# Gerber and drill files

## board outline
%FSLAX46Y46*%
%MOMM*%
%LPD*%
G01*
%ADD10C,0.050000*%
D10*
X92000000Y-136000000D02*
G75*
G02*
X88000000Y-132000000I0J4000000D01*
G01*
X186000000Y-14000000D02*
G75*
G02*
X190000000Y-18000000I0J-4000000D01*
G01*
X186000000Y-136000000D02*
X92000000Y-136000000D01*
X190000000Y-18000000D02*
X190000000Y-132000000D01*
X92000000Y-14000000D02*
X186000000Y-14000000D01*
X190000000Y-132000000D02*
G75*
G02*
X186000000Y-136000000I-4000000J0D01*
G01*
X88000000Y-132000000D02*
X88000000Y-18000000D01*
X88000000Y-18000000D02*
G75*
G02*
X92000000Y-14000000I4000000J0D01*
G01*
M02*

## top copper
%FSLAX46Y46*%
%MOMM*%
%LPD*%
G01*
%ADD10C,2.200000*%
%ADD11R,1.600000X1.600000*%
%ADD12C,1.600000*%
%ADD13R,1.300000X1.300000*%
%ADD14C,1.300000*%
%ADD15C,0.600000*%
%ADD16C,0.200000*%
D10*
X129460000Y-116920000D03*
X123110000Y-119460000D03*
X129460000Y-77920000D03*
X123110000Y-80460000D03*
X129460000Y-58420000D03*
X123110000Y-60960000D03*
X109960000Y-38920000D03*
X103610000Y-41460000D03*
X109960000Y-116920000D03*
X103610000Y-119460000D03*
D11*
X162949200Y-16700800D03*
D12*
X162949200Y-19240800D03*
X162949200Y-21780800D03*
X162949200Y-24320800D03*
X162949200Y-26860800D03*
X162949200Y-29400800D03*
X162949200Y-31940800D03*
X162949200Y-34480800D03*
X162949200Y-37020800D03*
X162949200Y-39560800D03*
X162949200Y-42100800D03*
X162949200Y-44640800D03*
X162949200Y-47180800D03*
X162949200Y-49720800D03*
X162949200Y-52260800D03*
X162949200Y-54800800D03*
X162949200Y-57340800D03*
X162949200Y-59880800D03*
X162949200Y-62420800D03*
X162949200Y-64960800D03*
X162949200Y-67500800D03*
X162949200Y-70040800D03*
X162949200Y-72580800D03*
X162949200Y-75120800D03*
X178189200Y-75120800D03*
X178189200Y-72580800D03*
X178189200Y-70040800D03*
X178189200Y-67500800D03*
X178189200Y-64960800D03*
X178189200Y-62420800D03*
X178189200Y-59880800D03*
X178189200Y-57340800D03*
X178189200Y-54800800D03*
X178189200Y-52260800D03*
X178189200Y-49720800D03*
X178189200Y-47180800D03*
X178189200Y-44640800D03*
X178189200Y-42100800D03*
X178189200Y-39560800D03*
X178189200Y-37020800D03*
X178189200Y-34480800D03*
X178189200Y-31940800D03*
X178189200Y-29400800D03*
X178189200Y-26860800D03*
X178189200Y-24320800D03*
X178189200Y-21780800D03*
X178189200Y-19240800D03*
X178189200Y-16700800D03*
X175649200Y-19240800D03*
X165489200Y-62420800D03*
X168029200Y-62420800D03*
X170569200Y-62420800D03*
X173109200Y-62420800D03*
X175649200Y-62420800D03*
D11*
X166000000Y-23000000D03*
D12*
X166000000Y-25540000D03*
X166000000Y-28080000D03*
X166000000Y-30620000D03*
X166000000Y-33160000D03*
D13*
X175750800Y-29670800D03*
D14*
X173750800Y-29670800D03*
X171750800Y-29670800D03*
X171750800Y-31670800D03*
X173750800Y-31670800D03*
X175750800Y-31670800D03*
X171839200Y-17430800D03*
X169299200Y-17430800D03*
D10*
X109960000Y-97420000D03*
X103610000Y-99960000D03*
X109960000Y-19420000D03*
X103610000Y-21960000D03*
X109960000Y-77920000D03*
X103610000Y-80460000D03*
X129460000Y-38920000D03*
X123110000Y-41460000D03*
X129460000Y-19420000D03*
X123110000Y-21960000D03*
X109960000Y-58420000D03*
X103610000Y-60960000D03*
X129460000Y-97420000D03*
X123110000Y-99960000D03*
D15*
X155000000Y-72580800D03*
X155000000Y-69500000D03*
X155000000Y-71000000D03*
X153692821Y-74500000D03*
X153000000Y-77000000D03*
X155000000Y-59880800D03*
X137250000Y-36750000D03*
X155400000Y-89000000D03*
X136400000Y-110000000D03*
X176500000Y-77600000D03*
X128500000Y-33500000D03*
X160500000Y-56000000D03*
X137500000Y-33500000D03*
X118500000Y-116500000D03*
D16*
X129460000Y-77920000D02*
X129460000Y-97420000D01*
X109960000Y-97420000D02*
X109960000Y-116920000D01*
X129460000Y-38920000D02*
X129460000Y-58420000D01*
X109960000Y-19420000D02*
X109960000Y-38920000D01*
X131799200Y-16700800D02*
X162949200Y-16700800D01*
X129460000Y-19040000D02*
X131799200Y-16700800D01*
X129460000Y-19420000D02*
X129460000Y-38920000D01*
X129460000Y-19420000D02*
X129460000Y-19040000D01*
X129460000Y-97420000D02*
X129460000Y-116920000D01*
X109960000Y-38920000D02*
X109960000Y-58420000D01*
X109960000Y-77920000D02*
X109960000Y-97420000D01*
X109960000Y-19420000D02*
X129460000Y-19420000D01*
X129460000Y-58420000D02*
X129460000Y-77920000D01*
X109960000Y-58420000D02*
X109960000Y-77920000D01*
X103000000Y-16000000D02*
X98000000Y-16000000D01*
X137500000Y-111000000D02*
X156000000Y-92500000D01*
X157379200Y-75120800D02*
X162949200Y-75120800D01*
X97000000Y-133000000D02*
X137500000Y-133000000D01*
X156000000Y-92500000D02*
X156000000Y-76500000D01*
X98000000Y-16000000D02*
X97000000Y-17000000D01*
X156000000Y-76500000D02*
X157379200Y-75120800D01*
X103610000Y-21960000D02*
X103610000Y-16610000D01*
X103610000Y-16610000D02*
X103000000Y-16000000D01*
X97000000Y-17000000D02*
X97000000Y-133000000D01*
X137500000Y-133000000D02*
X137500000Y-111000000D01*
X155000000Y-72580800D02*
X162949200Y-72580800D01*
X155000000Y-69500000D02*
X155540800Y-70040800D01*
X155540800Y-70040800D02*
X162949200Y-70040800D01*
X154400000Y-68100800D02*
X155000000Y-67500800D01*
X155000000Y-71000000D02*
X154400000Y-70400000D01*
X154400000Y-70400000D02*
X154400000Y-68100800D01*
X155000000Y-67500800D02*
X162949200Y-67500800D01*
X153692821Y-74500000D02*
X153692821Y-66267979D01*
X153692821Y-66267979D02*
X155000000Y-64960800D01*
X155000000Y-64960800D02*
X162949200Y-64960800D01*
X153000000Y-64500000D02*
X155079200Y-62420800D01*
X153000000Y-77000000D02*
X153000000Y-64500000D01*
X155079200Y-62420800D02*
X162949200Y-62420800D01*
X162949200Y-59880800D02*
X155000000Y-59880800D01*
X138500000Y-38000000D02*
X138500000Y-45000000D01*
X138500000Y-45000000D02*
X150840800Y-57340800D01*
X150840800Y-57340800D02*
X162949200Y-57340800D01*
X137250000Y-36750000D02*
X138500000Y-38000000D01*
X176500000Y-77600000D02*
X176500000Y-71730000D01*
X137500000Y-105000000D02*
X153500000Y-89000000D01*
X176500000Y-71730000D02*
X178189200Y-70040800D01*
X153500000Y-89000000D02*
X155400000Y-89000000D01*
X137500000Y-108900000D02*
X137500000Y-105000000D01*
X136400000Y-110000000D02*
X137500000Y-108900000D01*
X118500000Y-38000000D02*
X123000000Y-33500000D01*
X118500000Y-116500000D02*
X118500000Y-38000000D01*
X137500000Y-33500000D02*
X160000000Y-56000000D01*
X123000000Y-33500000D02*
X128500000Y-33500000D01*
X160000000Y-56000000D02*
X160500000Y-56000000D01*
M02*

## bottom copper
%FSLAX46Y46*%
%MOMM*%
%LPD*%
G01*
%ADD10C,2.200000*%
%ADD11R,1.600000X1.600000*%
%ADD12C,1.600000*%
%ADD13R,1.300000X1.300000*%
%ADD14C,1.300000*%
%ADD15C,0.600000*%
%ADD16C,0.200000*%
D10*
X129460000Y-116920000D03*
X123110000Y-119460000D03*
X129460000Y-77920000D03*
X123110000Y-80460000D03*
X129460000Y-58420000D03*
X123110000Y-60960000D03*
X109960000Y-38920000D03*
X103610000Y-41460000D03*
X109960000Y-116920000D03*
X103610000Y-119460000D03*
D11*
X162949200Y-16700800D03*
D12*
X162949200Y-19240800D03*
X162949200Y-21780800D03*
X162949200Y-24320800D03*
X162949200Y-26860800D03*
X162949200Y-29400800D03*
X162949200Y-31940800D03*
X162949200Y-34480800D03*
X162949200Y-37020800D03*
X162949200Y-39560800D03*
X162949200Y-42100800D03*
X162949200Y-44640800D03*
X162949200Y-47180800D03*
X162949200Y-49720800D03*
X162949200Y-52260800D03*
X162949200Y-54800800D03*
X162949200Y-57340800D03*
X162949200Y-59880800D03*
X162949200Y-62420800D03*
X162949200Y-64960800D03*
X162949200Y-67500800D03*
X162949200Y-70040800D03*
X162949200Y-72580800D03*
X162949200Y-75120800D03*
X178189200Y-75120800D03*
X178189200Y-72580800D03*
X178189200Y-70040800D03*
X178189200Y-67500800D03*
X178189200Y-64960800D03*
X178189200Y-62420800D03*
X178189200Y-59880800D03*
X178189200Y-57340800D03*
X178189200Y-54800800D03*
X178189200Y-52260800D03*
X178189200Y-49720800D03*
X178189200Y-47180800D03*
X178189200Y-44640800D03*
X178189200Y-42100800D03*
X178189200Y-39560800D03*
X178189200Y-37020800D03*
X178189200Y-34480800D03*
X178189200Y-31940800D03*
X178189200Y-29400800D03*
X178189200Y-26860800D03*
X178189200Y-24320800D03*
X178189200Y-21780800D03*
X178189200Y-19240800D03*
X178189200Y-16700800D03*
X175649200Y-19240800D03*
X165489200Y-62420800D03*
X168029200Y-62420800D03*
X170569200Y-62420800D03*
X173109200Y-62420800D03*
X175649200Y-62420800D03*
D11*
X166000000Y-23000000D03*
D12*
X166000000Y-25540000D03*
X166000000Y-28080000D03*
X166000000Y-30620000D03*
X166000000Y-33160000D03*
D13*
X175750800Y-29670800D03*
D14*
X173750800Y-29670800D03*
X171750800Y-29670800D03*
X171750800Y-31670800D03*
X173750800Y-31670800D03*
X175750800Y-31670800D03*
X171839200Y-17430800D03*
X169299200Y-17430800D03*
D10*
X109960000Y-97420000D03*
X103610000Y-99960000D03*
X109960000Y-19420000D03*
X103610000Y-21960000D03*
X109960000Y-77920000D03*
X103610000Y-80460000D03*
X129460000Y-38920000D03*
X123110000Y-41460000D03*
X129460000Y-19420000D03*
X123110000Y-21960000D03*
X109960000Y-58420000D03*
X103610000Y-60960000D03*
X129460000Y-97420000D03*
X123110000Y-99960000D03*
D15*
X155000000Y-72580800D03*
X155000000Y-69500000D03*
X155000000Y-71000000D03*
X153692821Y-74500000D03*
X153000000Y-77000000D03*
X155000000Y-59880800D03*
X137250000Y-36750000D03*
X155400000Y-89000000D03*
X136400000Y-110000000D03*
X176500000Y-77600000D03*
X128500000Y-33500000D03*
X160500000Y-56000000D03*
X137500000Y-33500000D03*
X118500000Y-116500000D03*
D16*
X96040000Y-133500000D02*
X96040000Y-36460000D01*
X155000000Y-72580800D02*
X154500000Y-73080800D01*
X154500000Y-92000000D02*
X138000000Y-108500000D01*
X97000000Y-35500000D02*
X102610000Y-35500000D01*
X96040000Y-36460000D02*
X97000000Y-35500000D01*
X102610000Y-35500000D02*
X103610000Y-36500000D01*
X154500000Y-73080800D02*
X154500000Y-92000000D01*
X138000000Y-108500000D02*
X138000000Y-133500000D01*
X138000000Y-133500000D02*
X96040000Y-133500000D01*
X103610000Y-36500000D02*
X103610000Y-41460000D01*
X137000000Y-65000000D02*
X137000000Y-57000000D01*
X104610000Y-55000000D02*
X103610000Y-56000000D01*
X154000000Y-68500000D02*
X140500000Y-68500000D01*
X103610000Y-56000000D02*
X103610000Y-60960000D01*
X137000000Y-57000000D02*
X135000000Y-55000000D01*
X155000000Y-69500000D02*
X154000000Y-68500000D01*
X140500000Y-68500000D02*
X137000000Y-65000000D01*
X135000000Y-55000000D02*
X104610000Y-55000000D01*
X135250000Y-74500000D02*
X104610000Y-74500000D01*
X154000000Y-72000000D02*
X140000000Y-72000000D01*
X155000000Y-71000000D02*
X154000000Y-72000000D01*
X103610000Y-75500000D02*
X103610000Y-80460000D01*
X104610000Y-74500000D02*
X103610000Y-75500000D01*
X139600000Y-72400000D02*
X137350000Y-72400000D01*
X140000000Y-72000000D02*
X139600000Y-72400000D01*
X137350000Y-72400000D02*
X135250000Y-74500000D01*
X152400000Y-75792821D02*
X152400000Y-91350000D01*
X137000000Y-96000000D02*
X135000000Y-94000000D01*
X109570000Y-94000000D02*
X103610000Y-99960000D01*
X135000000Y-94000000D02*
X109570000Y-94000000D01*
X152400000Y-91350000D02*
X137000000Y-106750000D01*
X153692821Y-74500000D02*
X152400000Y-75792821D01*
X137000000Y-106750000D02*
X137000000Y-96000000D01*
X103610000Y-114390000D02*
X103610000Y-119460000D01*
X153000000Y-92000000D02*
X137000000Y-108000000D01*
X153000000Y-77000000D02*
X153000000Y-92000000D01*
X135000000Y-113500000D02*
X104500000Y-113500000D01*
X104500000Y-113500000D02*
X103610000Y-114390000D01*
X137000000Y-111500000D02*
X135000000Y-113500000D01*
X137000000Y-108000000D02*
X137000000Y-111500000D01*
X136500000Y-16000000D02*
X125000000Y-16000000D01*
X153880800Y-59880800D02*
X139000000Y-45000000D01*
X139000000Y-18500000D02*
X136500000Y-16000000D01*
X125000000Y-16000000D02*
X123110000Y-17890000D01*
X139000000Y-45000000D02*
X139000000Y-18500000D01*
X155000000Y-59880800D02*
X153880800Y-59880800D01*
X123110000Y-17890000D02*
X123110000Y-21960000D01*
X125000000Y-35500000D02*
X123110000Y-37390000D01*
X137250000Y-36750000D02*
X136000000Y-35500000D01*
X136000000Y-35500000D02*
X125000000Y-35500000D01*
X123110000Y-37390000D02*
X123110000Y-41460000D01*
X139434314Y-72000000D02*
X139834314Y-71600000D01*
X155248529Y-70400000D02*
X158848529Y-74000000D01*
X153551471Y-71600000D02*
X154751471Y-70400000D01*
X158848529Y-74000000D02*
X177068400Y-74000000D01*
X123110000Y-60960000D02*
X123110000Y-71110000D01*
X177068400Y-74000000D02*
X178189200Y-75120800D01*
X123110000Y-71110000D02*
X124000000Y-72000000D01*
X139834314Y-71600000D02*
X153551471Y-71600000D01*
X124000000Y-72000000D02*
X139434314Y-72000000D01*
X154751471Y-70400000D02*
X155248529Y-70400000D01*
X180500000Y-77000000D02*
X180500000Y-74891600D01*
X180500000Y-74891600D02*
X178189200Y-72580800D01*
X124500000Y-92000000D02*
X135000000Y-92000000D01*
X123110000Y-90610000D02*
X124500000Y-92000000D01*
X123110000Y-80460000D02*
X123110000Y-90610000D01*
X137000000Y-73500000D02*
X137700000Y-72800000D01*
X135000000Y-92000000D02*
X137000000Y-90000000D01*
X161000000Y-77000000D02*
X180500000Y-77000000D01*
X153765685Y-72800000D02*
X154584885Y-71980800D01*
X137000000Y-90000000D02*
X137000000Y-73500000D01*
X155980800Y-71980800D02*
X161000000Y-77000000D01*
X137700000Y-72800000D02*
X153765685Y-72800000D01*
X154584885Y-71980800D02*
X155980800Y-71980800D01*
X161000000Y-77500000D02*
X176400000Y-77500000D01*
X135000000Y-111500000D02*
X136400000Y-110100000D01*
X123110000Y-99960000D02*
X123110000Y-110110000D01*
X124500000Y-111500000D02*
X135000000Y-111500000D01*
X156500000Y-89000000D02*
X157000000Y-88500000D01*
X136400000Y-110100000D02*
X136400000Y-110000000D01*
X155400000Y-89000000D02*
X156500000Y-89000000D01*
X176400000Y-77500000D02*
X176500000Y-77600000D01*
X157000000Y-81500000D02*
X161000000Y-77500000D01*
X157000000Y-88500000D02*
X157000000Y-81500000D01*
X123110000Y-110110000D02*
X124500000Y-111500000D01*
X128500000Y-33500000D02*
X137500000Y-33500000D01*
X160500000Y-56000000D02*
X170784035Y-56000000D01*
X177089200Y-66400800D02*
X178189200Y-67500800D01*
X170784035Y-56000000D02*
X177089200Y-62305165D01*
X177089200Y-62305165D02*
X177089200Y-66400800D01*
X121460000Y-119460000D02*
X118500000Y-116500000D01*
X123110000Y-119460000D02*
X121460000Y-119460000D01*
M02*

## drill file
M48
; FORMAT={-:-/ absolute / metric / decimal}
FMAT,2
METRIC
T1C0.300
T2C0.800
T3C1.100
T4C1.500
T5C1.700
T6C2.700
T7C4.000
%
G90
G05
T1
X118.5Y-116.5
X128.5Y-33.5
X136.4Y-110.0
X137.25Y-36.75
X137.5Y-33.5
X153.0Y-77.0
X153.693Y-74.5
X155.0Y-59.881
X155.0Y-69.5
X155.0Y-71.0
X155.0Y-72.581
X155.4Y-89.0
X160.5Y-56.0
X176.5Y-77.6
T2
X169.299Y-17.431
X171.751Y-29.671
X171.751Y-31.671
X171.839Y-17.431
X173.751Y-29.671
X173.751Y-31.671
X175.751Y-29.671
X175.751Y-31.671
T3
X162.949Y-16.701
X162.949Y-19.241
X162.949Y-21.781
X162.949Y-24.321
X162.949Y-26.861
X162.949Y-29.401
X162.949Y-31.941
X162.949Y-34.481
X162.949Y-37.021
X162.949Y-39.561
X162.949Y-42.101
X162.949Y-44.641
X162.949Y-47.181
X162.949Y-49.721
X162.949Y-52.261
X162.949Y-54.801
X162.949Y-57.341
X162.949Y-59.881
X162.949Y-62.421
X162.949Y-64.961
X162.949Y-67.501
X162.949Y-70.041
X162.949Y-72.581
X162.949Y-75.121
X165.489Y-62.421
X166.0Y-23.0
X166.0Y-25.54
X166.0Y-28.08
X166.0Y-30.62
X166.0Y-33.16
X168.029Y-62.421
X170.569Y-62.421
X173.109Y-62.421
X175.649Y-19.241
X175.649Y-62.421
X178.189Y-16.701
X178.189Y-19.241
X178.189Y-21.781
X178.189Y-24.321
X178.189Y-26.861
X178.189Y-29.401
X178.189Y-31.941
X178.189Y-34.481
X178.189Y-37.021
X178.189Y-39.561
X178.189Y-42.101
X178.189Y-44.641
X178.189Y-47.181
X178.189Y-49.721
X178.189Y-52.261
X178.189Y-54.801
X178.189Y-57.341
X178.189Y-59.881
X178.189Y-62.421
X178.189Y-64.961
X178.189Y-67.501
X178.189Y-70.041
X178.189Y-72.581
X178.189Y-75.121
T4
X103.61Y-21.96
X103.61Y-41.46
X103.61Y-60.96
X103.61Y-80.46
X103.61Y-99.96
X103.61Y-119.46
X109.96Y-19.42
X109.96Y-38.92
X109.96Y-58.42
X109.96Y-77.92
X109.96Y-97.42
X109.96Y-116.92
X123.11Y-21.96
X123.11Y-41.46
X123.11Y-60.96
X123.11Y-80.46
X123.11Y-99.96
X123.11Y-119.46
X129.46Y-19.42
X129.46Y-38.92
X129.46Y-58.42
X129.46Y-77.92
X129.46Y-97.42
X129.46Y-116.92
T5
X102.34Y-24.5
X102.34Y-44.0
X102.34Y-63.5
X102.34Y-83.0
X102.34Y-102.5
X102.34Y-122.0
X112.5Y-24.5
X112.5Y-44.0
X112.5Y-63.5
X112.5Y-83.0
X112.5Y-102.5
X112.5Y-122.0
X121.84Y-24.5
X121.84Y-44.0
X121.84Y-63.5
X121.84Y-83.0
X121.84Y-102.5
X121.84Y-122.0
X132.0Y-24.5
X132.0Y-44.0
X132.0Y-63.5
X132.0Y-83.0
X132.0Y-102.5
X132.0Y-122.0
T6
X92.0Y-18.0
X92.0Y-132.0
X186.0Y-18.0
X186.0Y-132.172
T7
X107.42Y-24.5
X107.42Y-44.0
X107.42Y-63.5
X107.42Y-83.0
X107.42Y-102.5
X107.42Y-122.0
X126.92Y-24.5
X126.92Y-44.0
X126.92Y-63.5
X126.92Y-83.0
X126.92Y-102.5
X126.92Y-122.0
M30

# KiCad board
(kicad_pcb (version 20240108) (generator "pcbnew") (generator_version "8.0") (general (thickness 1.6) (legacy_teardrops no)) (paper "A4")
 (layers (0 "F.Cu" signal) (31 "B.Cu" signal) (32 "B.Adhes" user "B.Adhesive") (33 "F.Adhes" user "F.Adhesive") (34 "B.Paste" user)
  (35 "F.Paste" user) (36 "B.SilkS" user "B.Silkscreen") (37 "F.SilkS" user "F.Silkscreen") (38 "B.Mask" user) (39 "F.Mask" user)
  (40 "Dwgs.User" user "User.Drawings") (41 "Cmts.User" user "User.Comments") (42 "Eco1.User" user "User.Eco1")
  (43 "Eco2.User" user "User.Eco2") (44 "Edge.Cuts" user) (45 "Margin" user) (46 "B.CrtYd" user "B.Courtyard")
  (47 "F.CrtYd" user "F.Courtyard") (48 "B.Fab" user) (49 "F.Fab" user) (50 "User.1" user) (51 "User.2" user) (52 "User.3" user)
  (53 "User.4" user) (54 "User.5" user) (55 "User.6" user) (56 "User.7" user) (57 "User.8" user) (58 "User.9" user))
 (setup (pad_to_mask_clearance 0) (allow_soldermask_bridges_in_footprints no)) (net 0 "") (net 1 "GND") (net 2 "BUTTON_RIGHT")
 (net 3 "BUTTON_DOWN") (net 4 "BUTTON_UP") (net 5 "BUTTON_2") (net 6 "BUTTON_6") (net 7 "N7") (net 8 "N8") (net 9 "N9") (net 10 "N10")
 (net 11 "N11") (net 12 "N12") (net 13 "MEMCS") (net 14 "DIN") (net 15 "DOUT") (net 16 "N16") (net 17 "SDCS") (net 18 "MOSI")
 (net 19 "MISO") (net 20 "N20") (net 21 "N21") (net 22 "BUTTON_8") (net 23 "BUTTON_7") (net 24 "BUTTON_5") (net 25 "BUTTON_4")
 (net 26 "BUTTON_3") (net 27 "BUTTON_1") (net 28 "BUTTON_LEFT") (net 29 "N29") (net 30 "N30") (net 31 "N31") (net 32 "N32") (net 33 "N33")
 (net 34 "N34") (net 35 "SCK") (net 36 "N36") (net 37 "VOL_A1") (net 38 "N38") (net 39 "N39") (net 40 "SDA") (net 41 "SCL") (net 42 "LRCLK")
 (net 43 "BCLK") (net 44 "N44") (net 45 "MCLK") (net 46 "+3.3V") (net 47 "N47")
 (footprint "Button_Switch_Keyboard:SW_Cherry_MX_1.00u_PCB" (layer "F.Cu") (at 129.46 116.92)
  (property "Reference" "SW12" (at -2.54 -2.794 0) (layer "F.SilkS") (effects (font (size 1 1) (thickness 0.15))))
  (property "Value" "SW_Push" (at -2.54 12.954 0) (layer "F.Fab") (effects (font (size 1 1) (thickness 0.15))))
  (pad "" np_thru_hole circle (at -7.62 5.08) (size 1.7 1.7) (drill 1.7) (layers "*.Cu" "*.Mask"))
  (pad "" np_thru_hole circle (at -2.54 5.08) (size 4 4) (drill 4) (layers "*.Cu" "*.Mask"))
  (pad "" np_thru_hole circle (at 2.54 5.08) (size 1.7 1.7) (drill 1.7) (layers "*.Cu" "*.Mask"))
  (pad "1" thru_hole circle (at 0 0) (size 2.2 2.2) (drill 1.5) (layers "*.Cu" "*.Mask") (remove_unused_layers no) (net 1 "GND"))
  (pad "2" thru_hole circle (at -6.35 2.54) (size 2.2 2.2) (drill 1.5) (layers "*.Cu" "*.Mask") (remove_unused_layers no)
   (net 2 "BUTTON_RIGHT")))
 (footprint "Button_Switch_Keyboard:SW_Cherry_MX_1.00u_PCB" (layer "F.Cu") (at 129.46 77.92)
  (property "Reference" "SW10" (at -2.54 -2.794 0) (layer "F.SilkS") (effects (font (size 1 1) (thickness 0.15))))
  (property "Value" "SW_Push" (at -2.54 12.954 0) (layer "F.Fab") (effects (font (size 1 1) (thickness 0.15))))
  (pad "" np_thru_hole circle (at -7.62 5.08) (size 1.7 1.7) (drill 1.7) (layers "*.Cu" "*.Mask"))
  (pad "" np_thru_hole circle (at -2.54 5.08) (size 4 4) (drill 4) (layers "*.Cu" "*.Mask"))
  (pad "" np_thru_hole circle (at 2.54 5.08) (size 1.7 1.7) (drill 1.7) (layers "*.Cu" "*.Mask"))
  (pad "1" thru_hole circle (at 0 0) (size 2.2 2.2) (drill 1.5) (layers "*.Cu" "*.Mask") (remove_unused_layers no) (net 1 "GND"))
  (pad "2" thru_hole circle (at -6.35 2.54) (size 2.2 2.2) (drill 1.5) (layers "*.Cu" "*.Mask") (remove_unused_layers no)
   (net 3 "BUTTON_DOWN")))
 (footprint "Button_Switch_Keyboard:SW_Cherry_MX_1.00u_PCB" (layer "F.Cu") (at 129.46 58.42)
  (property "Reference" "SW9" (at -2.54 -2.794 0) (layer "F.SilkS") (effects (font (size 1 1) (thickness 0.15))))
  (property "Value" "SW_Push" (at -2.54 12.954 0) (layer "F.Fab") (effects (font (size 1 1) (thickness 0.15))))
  (pad "" np_thru_hole circle (at -7.62 5.08) (size 1.7 1.7) (drill 1.7) (layers "*.Cu" "*.Mask"))
  (pad "" np_thru_hole circle (at -2.54 5.08) (size 4 4) (drill 4) (layers "*.Cu" "*.Mask"))
  (pad "" np_thru_hole circle (at 2.54 5.08) (size 1.7 1.7) (drill 1.7) (layers "*.Cu" "*.Mask"))
  (pad "1" thru_hole circle (at 0 0) (size 2.2 2.2) (drill 1.5) (layers "*.Cu" "*.Mask") (remove_unused_layers no) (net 1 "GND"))
  (pad "2" thru_hole circle (at -6.35 2.54) (size 2.2 2.2) (drill 1.5) (layers "*.Cu" "*.Mask") (remove_unused_layers no)
   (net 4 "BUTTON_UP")))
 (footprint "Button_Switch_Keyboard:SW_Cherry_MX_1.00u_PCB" (layer "F.Cu") (at 109.96 38.92)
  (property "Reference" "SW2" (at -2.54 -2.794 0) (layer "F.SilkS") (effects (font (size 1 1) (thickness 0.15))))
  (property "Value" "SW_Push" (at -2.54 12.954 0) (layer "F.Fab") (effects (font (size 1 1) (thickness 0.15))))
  (pad "" np_thru_hole circle (at -7.62 5.08) (size 1.7 1.7) (drill 1.7) (layers "*.Cu" "*.Mask"))
  (pad "" np_thru_hole circle (at -2.54 5.08) (size 4 4) (drill 4) (layers "*.Cu" "*.Mask"))
  (pad "" np_thru_hole circle (at 2.54 5.08) (size 1.7 1.7) (drill 1.7) (layers "*.Cu" "*.Mask"))
  (pad "1" thru_hole circle (at 0 0) (size 2.2 2.2) (drill 1.5) (layers "*.Cu" "*.Mask") (remove_unused_layers no) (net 1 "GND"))
  (pad "2" thru_hole circle (at -6.35 2.54) (size 2.2 2.2) (drill 1.5) (layers "*.Cu" "*.Mask") (remove_unused_layers no) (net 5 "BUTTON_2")))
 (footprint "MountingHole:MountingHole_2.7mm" (layer "F.Cu") (at 92 18)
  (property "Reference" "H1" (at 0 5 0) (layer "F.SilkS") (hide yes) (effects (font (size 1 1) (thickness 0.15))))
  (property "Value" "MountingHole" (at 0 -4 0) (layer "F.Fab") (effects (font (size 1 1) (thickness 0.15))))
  (pad "" np_thru_hole circle (at 0 0) (size 2.7 2.7) (drill 2.7) (layers "*.Cu" "*.Mask")))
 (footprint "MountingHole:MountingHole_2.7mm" (layer "F.Cu") (at 186 18)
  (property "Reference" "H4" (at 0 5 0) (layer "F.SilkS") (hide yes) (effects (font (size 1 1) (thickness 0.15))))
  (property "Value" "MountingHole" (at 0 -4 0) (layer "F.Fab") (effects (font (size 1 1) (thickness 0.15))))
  (pad "" np_thru_hole circle (at 0 0) (size 2.7 2.7) (drill 2.7) (layers "*.Cu" "*.Mask")))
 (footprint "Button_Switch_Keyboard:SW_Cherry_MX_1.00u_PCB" (layer "F.Cu") (at 109.96 116.92)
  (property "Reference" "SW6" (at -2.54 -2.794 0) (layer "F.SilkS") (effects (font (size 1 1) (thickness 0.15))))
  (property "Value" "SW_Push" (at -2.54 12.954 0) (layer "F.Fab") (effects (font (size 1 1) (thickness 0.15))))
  (pad "" np_thru_hole circle (at -7.62 5.08) (size 1.7 1.7) (drill 1.7) (layers "*.Cu" "*.Mask"))
  (pad "" np_thru_hole circle (at -2.54 5.08) (size 4 4) (drill 4) (layers "*.Cu" "*.Mask"))
  (pad "" np_thru_hole circle (at 2.54 5.08) (size 1.7 1.7) (drill 1.7) (layers "*.Cu" "*.Mask"))
  (pad "1" thru_hole circle (at 0 0) (size 2.2 2.2) (drill 1.5) (layers "*.Cu" "*.Mask") (remove_unused_layers no) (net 1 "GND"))
  (pad "2" thru_hole circle (at -6.35 2.54) (size 2.2 2.2) (drill 1.5) (layers "*.Cu" "*.Mask") (remove_unused_layers no) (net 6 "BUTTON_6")))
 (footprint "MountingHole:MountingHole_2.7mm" (layer "F.Cu") (at 186 132.171573)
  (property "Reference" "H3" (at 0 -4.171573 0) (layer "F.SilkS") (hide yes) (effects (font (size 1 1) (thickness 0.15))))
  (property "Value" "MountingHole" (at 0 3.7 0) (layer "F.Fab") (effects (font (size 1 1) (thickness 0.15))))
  (pad "" np_thru_hole circle (at 0 0) (size 2.7 2.7) (drill 2.7) (layers "*.Cu" "*.Mask")))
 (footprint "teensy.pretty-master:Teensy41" (layer "F.Cu") (at 170.5692 45.9108 -90)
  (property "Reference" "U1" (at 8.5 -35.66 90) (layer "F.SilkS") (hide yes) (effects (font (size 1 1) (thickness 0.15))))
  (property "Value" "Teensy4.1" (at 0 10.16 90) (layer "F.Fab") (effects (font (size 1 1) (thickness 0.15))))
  (pad "1" thru_hole rect (at -29.21 7.62 270) (size 1.6 1.6) (drill 1.1) (layers "*.Cu" "*.Mask") (remove_unused_layers no) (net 1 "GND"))
  (pad "2" thru_hole circle (at -26.67 7.62 270) (size 1.6 1.6) (drill 1.1) (layers "*.Cu" "*.Mask") (remove_unused_layers no) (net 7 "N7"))
  (pad "3" thru_hole circle (at -24.13 7.62 270) (size 1.6 1.6) (drill 1.1) (layers "*.Cu" "*.Mask") (remove_unused_layers no) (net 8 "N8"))
  (pad "4" thru_hole circle (at -21.59 7.62 270) (size 1.6 1.6) (drill 1.1) (layers "*.Cu" "*.Mask") (remove_unused_layers no) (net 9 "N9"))
  (pad "5" thru_hole circle (at -19.05 7.62 270) (size 1.6 1.6) (drill 1.1) (layers "*.Cu" "*.Mask") (remove_unused_layers no)
   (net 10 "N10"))
  (pad "6" thru_hole circle (at -16.51 7.62 270) (size 1.6 1.6) (drill 1.1) (layers "*.Cu" "*.Mask") (remove_unused_layers no)
   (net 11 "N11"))
  (pad "7" thru_hole circle (at -13.97 7.62 270) (size 1.6 1.6) (drill 1.1) (layers "*.Cu" "*.Mask") (remove_unused_layers no)
   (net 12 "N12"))
  (pad "8" thru_hole circle (at -11.43 7.62 270) (size 1.6 1.6) (drill 1.1) (layers "*.Cu" "*.Mask") (remove_unused_layers no)
   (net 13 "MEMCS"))
  (pad "9" thru_hole circle (at -8.89 7.62 270) (size 1.6 1.6) (drill 1.1) (layers "*.Cu" "*.Mask") (remove_unused_layers no) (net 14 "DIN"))
  (pad "10" thru_hole circle (at -6.35 7.62 270) (size 1.6 1.6) (drill 1.1) (layers "*.Cu" "*.Mask") (remove_unused_layers no)
   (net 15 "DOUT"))
  (pad "11" thru_hole circle (at -3.81 7.62 270) (size 1.6 1.6) (drill 1.1) (layers "*.Cu" "*.Mask") (remove_unused_layers no)
   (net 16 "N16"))
  (pad "12" thru_hole circle (at -1.27 7.62 270) (size 1.6 1.6) (drill 1.1) (layers "*.Cu" "*.Mask") (remove_unused_layers no)
   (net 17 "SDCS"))
  (pad "13" thru_hole circle (at 1.27 7.62 270) (size 1.6 1.6) (drill 1.1) (layers "*.Cu" "*.Mask") (remove_unused_layers no)
   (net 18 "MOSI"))
  (pad "14" thru_hole circle (at 3.81 7.62 270) (size 1.6 1.6) (drill 1.1) (layers "*.Cu" "*.Mask") (remove_unused_layers no)
   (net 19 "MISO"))
  (pad "15" thru_hole circle (at 6.35 7.62 270) (size 1.6 1.6) (drill 1.1) (layers "*.Cu" "*.Mask") (remove_unused_layers no) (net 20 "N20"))
  (pad "16" thru_hole circle (at 8.89 7.62 270) (size 1.6 1.6) (drill 1.1) (layers "*.Cu" "*.Mask") (remove_unused_layers no) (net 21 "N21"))
  (pad "17" thru_hole circle (at 11.43 7.62 270) (size 1.6 1.6) (drill 1.1) (layers "*.Cu" "*.Mask") (remove_unused_layers no)
   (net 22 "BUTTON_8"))
  (pad "18" thru_hole circle (at 13.97 7.62 270) (size 1.6 1.6) (drill 1.1) (layers "*.Cu" "*.Mask") (remove_unused_layers no)
   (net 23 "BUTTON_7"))
  (pad "19" thru_hole circle (at 16.51 7.62 270) (size 1.6 1.6) (drill 1.1) (layers "*.Cu" "*.Mask") (remove_unused_layers no)
   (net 6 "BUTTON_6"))
  (pad "20" thru_hole circle (at 19.05 7.62 270) (size 1.6 1.6) (drill 1.1) (layers "*.Cu" "*.Mask") (remove_unused_layers no)
   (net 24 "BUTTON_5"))
  (pad "21" thru_hole circle (at 21.59 7.62 270) (size 1.6 1.6) (drill 1.1) (layers "*.Cu" "*.Mask") (remove_unused_layers no)
   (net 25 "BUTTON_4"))
  (pad "22" thru_hole circle (at 24.13 7.62 270) (size 1.6 1.6) (drill 1.1) (layers "*.Cu" "*.Mask") (remove_unused_layers no)
   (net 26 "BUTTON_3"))
  (pad "23" thru_hole circle (at 26.67 7.62 270) (size 1.6 1.6) (drill 1.1) (layers "*.Cu" "*.Mask") (remove_unused_layers no)
   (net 5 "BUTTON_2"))
  (pad "24" thru_hole circle (at 29.21 7.62 270) (size 1.6 1.6) (drill 1.1) (layers "*.Cu" "*.Mask") (remove_unused_layers no)
   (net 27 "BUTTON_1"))
  (pad "25" thru_hole circle (at 29.21 -7.62 270) (size 1.6 1.6) (drill 1.1) (layers "*.Cu" "*.Mask") (remove_unused_layers no)
   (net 4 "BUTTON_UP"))
  (pad "26" thru_hole circle (at 26.67 -7.62 270) (size 1.6 1.6) (drill 1.1) (layers "*.Cu" "*.Mask") (remove_unused_layers no)
   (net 3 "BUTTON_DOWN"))
  (pad "27" thru_hole circle (at 24.13 -7.62 270) (size 1.6 1.6) (drill 1.1) (layers "*.Cu" "*.Mask") (remove_unused_layers no)
   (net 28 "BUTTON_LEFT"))
  (pad "28" thru_hole circle (at 21.59 -7.62 270) (size 1.6 1.6) (drill 1.1) (layers "*.Cu" "*.Mask") (remove_unused_layers no)
   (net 2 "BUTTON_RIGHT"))
  (pad "29" thru_hole circle (at 19.05 -7.62 270) (size 1.6 1.6) (drill 1.1) (layers "*.Cu" "*.Mask") (remove_unused_layers no)
   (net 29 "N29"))
  (pad "30" thru_hole circle (at 16.51 -7.62 270) (size 1.6 1.6) (drill 1.1) (layers "*.Cu" "*.Mask") (remove_unused_layers no)
   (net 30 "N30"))
  (pad "31" thru_hole circle (at 13.97 -7.62 270) (size 1.6 1.6) (drill 1.1) (layers "*.Cu" "*.Mask") (remove_unused_layers no)
   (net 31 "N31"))
  (pad "32" thru_hole circle (at 11.43 -7.62 270) (size 1.6 1.6) (drill 1.1) (layers "*.Cu" "*.Mask") (remove_unused_layers no)
   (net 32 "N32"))
  (pad "33" thru_hole circle (at 8.89 -7.62 270) (size 1.6 1.6) (drill 1.1) (layers "*.Cu" "*.Mask") (remove_unused_layers no)
   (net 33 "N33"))
  (pad "34" thru_hole circle (at 6.35 -7.62 270) (size 1.6 1.6) (drill 1.1) (layers "*.Cu" "*.Mask") (remove_unused_layers no)
   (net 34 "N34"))
  (pad "35" thru_hole circle (at 3.81 -7.62 270) (size 1.6 1.6) (drill 1.1) (layers "*.Cu" "*.Mask") (remove_unused_layers no)
   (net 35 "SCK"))
  (pad "36" thru_hole circle (at 1.27 -7.62 270) (size 1.6 1.6) (drill 1.1) (layers "*.Cu" "*.Mask") (remove_unused_layers no)
   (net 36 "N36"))
  (pad "37" thru_hole circle (at -1.27 -7.62 270) (size 1.6 1.6) (drill 1.1) (layers "*.Cu" "*.Mask") (remove_unused_layers no)
   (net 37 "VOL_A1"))
  (pad "38" thru_hole circle (at -3.81 -7.62 270) (size 1.6 1.6) (drill 1.1) (layers "*.Cu" "*.Mask") (remove_unused_layers no)
   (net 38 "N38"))
  (pad "39" thru_hole circle (at -6.35 -7.62 270) (size 1.6 1.6) (drill 1.1) (layers "*.Cu" "*.Mask") (remove_unused_layers no)
   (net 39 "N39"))
  (pad "40" thru_hole circle (at -8.89 -7.62 270) (size 1.6 1.6) (drill 1.1) (layers "*.Cu" "*.Mask") (remove_unused_layers no)
   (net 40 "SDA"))
  (pad "41" thru_hole circle (at -11.43 -7.62 270) (size 1.6 1.6) (drill 1.1) (layers "*.Cu" "*.Mask") (remove_unused_layers no)
   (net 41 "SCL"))
  (pad "42" thru_hole circle (at -13.97 -7.62 270) (size 1.6 1.6) (drill 1.1) (layers "*.Cu" "*.Mask") (remove_unused_layers no)
   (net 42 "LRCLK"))
  (pad "43" thru_hole circle (at -16.51 -7.62 270) (size 1.6 1.6) (drill 1.1) (layers "*.Cu" "*.Mask") (remove_unused_layers no)
   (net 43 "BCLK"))
  (pad "44" thru_hole circle (at -19.05 -7.62 270) (size 1.6 1.6) (drill 1.1) (layers "*.Cu" "*.Mask") (remove_unused_layers no)
   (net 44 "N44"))
  (pad "45" thru_hole circle (at -21.59 -7.62 270) (size 1.6 1.6) (drill 1.1) (layers "*.Cu" "*.Mask") (remove_unused_layers no)
   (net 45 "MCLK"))
  (pad "46" thru_hole circle (at -24.13 -7.62 270) (size 1.6 1.6) (drill 1.1) (layers "*.Cu" "*.Mask") (remove_unused_layers no)
   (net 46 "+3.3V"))
  (pad "47" thru_hole circle (at -26.67 -7.62 270) (size 1.6 1.6) (drill 1.1) (layers "*.Cu" "*.Mask") (remove_unused_layers no)
   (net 1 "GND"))
  (pad "48" thru_hole circle (at -29.21 -7.62 270) (size 1.6 1.6) (drill 1.1) (layers "*.Cu" "*.Mask") (remove_unused_layers no)
   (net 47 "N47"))
  (pad "49" thru_hole circle (at -26.67 -5.08 270) (size 1.6 1.6) (drill 1.1) (layers "*.Cu" "*.Mask") (remove_unused_layers no))
  (pad "50" thru_hole circle (at 16.51 5.08 270) (size 1.6 1.6) (drill 1.1) (layers "*.Cu" "*.Mask") (remove_unused_layers no))
  (pad "51" thru_hole circle (at 16.51 2.54 270) (size 1.6 1.6) (drill 1.1) (layers "*.Cu" "*.Mask") (remove_unused_layers no))
  (pad "52" thru_hole circle (at 16.51 0 270) (size 1.6 1.6) (drill 1.1) (layers "*.Cu" "*.Mask") (remove_unused_layers no))
  (pad "53" thru_hole circle (at 16.51 -2.54 270) (size 1.6 1.6) (drill 1.1) (layers "*.Cu" "*.Mask") (remove_unused_layers no))
  (pad "54" thru_hole circle (at 16.51 -5.08 270) (size 1.6 1.6) (drill 1.1) (layers "*.Cu" "*.Mask") (remove_unused_layers no))
  (pad "55" thru_hole rect (at -22.9108 4.5692 270) (size 1.6 1.6) (drill 1.1) (layers "*.Cu" "*.Mask") (remove_unused_layers no))
  (pad "56" thru_hole circle (at -20.3708 4.5692 270) (size 1.6 1.6) (drill 1.1) (layers "*.Cu" "*.Mask") (remove_unused_layers no))
  (pad "57" thru_hole circle (at -17.8308 4.5692 270) (size 1.6 1.6) (drill 1.1) (layers "*.Cu" "*.Mask") (remove_unused_layers no))
  (pad "58" thru_hole circle (at -15.2908 4.5692 270) (size 1.6 1.6) (drill 1.1) (layers "*.Cu" "*.Mask") (remove_unused_layers no))
  (pad "59" thru_hole circle (at -12.7508 4.5692 270) (size 1.6 1.6) (drill 1.1) (layers "*.Cu" "*.Mask") (remove_unused_layers no))
  (pad "60" thru_hole rect (at -16.24 -5.1816 270) (size 1.3 1.3) (drill 0.8) (layers "*.Cu" "*.Mask") (remove_unused_layers no))
  (pad "61" thru_hole circle (at -16.24 -3.1816 270) (size 1.3 1.3) (drill 0.8) (layers "*.Cu" "*.Mask") (remove_unused_layers no))
  (pad "62" thru_hole circle (at -16.24 -1.1816 270) (size 1.3 1.3) (drill 0.8) (layers "*.Cu" "*.Mask") (remove_unused_layers no))
  (pad "63" thru_hole circle (at -14.24 -1.1816 270) (size 1.3 1.3) (drill 0.8) (layers "*.Cu" "*.Mask") (remove_unused_layers no))
  (pad "64" thru_hole circle (at -14.24 -3.1816 270) (size 1.3 1.3) (drill 0.8) (layers "*.Cu" "*.Mask") (remove_unused_layers no))
  (pad "65" thru_hole circle (at -14.24 -5.1816 270) (size 1.3 1.3) (drill 0.8) (layers "*.Cu" "*.Mask") (remove_unused_layers no))
  (pad "66" thru_hole circle (at -28.48 -1.27 270) (size 1.3 1.3) (drill 0.8) (layers "*.Cu" "*.Mask") (remove_unused_layers no))
  (pad "67" thru_hole circle (at -28.48 1.27 270) (size 1.3 1.3) (drill 0.8) (layers "*.Cu" "*.Mask") (remove_unused_layers no)))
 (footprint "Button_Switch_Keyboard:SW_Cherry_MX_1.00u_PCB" (layer "F.Cu") (at 109.96 97.42)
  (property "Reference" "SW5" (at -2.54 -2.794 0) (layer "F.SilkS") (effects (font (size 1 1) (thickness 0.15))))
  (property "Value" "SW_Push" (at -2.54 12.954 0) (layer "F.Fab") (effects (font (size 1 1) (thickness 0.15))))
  (pad "" np_thru_hole circle (at -7.62 5.08) (size 1.7 1.7) (drill 1.7) (layers "*.Cu" "*.Mask"))
  (pad "" np_thru_hole circle (at -2.54 5.08) (size 4 4) (drill 4) (layers "*.Cu" "*.Mask"))
  (pad "" np_thru_hole circle (at 2.54 5.08) (size 1.7 1.7) (drill 1.7) (layers "*.Cu" "*.Mask"))
  (pad "1" thru_hole circle (at 0 0) (size 2.2 2.2) (drill 1.5) (layers "*.Cu" "*.Mask") (remove_unused_layers no) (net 1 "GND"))
  (pad "2" thru_hole circle (at -6.35 2.54) (size 2.2 2.2) (drill 1.5) (layers "*.Cu" "*.Mask") (remove_unused_layers no)
   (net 24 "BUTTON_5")))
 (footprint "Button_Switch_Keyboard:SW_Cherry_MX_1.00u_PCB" (layer "F.Cu") (at 109.96 19.42)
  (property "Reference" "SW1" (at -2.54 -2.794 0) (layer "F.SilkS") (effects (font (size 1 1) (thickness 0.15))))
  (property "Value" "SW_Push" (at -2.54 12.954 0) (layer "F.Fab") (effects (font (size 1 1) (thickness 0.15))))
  (pad "" np_thru_hole circle (at -7.62 5.08) (size 1.7 1.7) (drill 1.7) (layers "*.Cu" "*.Mask"))
  (pad "" np_thru_hole circle (at -2.54 5.08) (size 4 4) (drill 4) (layers "*.Cu" "*.Mask"))
  (pad "" np_thru_hole circle (at 2.54 5.08) (size 1.7 1.7) (drill 1.7) (layers "*.Cu" "*.Mask"))
  (pad "1" thru_hole circle (at 0 0) (size 2.2 2.2) (drill 1.5) (layers "*.Cu" "*.Mask") (remove_unused_layers no) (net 1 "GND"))
  (pad "2" thru_hole circle (at -6.35 2.54) (size 2.2 2.2) (drill 1.5) (layers "*.Cu" "*.Mask") (remove_unused_layers no)
   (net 27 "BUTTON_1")))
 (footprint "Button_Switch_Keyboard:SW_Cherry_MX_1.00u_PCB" (layer "F.Cu") (at 109.96 77.92)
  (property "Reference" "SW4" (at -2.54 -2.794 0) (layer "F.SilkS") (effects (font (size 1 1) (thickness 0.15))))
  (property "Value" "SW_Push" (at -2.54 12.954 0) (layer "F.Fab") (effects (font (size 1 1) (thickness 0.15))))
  (pad "" np_thru_hole circle (at -7.62 5.08) (size 1.7 1.7) (drill 1.7) (layers "*.Cu" "*.Mask"))
  (pad "" np_thru_hole circle (at -2.54 5.08) (size 4 4) (drill 4) (layers "*.Cu" "*.Mask"))
  (pad "" np_thru_hole circle (at 2.54 5.08) (size 1.7 1.7) (drill 1.7) (layers "*.Cu" "*.Mask"))
  (pad "1" thru_hole circle (at 0 0) (size 2.2 2.2) (drill 1.5) (layers "*.Cu" "*.Mask") (remove_unused_layers no) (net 1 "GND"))
  (pad "2" thru_hole circle (at -6.35 2.54) (size 2.2 2.2) (drill 1.5) (layers "*.Cu" "*.Mask") (remove_unused_layers no)
   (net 25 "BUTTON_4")))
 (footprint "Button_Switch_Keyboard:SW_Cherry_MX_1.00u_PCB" (layer "F.Cu") (at 129.46 38.92)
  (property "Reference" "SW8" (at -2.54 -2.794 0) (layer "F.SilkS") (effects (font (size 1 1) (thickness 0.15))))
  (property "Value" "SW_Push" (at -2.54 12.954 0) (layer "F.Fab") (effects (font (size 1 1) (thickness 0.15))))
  (pad "" np_thru_hole circle (at -7.62 5.08) (size 1.7 1.7) (drill 1.7) (layers "*.Cu" "*.Mask"))
  (pad "" np_thru_hole circle (at -2.54 5.08) (size 4 4) (drill 4) (layers "*.Cu" "*.Mask"))
  (pad "" np_thru_hole circle (at 2.54 5.08) (size 1.7 1.7) (drill 1.7) (layers "*.Cu" "*.Mask"))
  (pad "1" thru_hole circle (at 0 0) (size 2.2 2.2) (drill 1.5) (layers "*.Cu" "*.Mask") (remove_unused_layers no) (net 1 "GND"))
  (pad "2" thru_hole circle (at -6.35 2.54) (size 2.2 2.2) (drill 1.5) (layers "*.Cu" "*.Mask") (remove_unused_layers no)
   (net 22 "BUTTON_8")))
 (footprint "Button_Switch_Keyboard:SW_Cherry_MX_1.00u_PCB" (layer "F.Cu") (at 129.46 19.42)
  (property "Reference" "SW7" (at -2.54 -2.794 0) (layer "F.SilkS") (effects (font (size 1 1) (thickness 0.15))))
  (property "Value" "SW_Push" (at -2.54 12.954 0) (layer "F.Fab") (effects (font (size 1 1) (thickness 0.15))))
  (pad "" np_thru_hole circle (at -7.62 5.08) (size 1.7 1.7) (drill 1.7) (layers "*.Cu" "*.Mask"))
  (pad "" np_thru_hole circle (at -2.54 5.08) (size 4 4) (drill 4) (layers "*.Cu" "*.Mask"))
  (pad "" np_thru_hole circle (at 2.54 5.08) (size 1.7 1.7) (drill 1.7) (layers "*.Cu" "*.Mask"))
  (pad "1" thru_hole circle (at 0 0) (size 2.2 2.2) (drill 1.5) (layers "*.Cu" "*.Mask") (remove_unused_layers no) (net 1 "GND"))
  (pad "2" thru_hole circle (at -6.35 2.54) (size 2.2 2.2) (drill 1.5) (layers "*.Cu" "*.Mask") (remove_unused_layers no)
   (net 23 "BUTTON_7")))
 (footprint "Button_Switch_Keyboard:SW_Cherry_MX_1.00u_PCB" (layer "F.Cu") (at 109.96 58.42)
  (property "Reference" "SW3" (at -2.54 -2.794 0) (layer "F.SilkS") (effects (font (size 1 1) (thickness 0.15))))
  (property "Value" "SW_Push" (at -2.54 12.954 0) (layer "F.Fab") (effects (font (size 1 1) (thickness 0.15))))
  (pad "" np_thru_hole circle (at -7.62 5.08) (size 1.7 1.7) (drill 1.7) (layers "*.Cu" "*.Mask"))
  (pad "" np_thru_hole circle (at -2.54 5.08) (size 4 4) (drill 4) (layers "*.Cu" "*.Mask"))
  (pad "" np_thru_hole circle (at 2.54 5.08) (size 1.7 1.7) (drill 1.7) (layers "*.Cu" "*.Mask"))
  (pad "1" thru_hole circle (at 0 0) (size 2.2 2.2) (drill 1.5) (layers "*.Cu" "*.Mask") (remove_unused_layers no) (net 1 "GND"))
  (pad "2" thru_hole circle (at -6.35 2.54) (size 2.2 2.2) (drill 1.5) (layers "*.Cu" "*.Mask") (remove_unused_layers no)
   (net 26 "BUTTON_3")))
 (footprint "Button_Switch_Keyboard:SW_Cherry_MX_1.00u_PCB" (layer "F.Cu") (at 129.46 97.42)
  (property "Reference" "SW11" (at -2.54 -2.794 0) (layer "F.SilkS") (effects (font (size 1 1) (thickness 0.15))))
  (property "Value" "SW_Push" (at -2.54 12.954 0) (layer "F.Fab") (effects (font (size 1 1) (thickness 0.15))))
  (pad "" np_thru_hole circle (at -7.62 5.08) (size 1.7 1.7) (drill 1.7) (layers "*.Cu" "*.Mask"))
  (pad "" np_thru_hole circle (at -2.54 5.08) (size 4 4) (drill 4) (layers "*.Cu" "*.Mask"))
  (pad "" np_thru_hole circle (at 2.54 5.08) (size 1.7 1.7) (drill 1.7) (layers "*.Cu" "*.Mask"))
  (pad "1" thru_hole circle (at 0 0) (size 2.2 2.2) (drill 1.5) (layers "*.Cu" "*.Mask") (remove_unused_layers no) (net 1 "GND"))
  (pad "2" thru_hole circle (at -6.35 2.54) (size 2.2 2.2) (drill 1.5) (layers "*.Cu" "*.Mask") (remove_unused_layers no)
   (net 28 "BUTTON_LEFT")))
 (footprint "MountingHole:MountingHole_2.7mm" (layer "F.Cu") (at 92 132)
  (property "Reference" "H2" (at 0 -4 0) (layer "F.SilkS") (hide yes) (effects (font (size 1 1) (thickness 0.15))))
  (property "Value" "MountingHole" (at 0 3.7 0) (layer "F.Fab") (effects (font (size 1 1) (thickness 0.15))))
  (pad "" np_thru_hole circle (at 0 0) (size 2.7 2.7) (drill 2.7) (layers "*.Cu" "*.Mask")))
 (gr_arc (start 92 136) (mid 89.171573 134.828427) (end 88 132) (stroke (width 0.05) (type default)) (layer "Edge.Cuts"))
 (gr_arc (start 186 14) (mid 188.828427 15.171573) (end 190 18) (stroke (width 0.05) (type default)) (layer "Edge.Cuts"))
 (gr_line (start 186 136) (end 92 136) (stroke (width 0.05) (type default)) (layer "Edge.Cuts"))
 (gr_line (start 190 18) (end 190 132) (stroke (width 0.05) (type default)) (layer "Edge.Cuts"))
 (gr_line (start 92 14) (end 186 14) (stroke (width 0.05) (type default)) (layer "Edge.Cuts"))
 (gr_arc (start 190 132) (mid 188.828427 134.828427) (end 186 136) (stroke (width 0.05) (type default)) (layer "Edge.Cuts"))
 (gr_line (start 88 132) (end 88 18) (stroke (width 0.05) (type default)) (layer "Edge.Cuts"))
 (gr_arc (start 88 18) (mid 89.171573 15.171573) (end 92 14) (stroke (width 0.05) (type default)) (layer "Edge.Cuts"))
 (segment (start 129.46 77.92) (end 129.46 97.42) (width 0.2) (layer "F.Cu") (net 1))
 (segment (start 109.96 97.42) (end 109.96 116.92) (width 0.2) (layer "F.Cu") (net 1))
 (segment (start 129.46 38.92) (end 129.46 58.42) (width 0.2) (layer "F.Cu") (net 1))
 (segment (start 109.96 19.42) (end 109.96 38.92) (width 0.2) (layer "F.Cu") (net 1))
 (segment (start 131.7992 16.7008) (end 162.9492 16.7008) (width 0.2) (layer "F.Cu") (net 1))
 (segment (start 129.46 19.04) (end 131.7992 16.7008) (width 0.2) (layer "F.Cu") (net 1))
 (segment (start 129.46 19.42) (end 129.46 38.92) (width 0.2) (layer "F.Cu") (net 1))
 (segment (start 129.46 19.42) (end 129.46 19.04) (width 0.2) (layer "F.Cu") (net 1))
 (segment (start 129.46 97.42) (end 129.46 116.92) (width 0.2) (layer "F.Cu") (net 1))
 (segment (start 109.96 38.92) (end 109.96 58.42) (width 0.2) (layer "F.Cu") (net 1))
 (segment (start 109.96 77.92) (end 109.96 97.42) (width 0.2) (layer "F.Cu") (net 1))
 (segment (start 109.96 19.42) (end 129.46 19.42) (width 0.2) (layer "F.Cu") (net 1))
 (segment (start 129.46 58.42) (end 129.46 77.92) (width 0.2) (layer "F.Cu") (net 1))
 (segment (start 109.96 58.42) (end 109.96 77.92) (width 0.2) (layer "F.Cu") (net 1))
 (segment (start 103 16) (end 98 16) (width 0.2) (layer "F.Cu") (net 27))
 (segment (start 137.5 111) (end 156 92.5) (width 0.2) (layer "F.Cu") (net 27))
 (segment (start 157.3792 75.1208) (end 162.9492 75.1208) (width 0.2) (layer "F.Cu") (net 27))
 (segment (start 97 133) (end 137.5 133) (width 0.2) (layer "F.Cu") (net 27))
 (segment (start 156 92.5) (end 156 76.5) (width 0.2) (layer "F.Cu") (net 27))
 (segment (start 98 16) (end 97 17) (width 0.2) (layer "F.Cu") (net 27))
 (segment (start 156 76.5) (end 157.3792 75.1208) (width 0.2) (layer "F.Cu") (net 27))
 (segment (start 103.61 21.96) (end 103.61 16.61) (width 0.2) (layer "F.Cu") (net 27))
 (segment (start 103.61 16.61) (end 103 16) (width 0.2) (layer "F.Cu") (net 27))
 (segment (start 97 17) (end 97 133) (width 0.2) (layer "F.Cu") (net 27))
 (segment (start 137.5 133) (end 137.5 111) (width 0.2) (layer "F.Cu") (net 27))
 (segment (start 155 72.5808) (end 162.9492 72.5808) (width 0.2) (layer "F.Cu") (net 5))
 (via (at 155 72.5808) (size 0.6) (drill 0.3) (layers "F.Cu" "B.Cu") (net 5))
 (segment (start 96.04 133.5) (end 96.04 36.46) (width 0.2) (layer "B.Cu") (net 5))
 (segment (start 155 72.5808) (end 154.5 73.0808) (width 0.2) (layer "B.Cu") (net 5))
 (segment (start 154.5 92) (end 138 108.5) (width 0.2) (layer "B.Cu") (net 5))
 (segment (start 97 35.5) (end 102.61 35.5) (width 0.2) (layer "B.Cu") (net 5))
 (segment (start 96.04 36.46) (end 97 35.5) (width 0.2) (layer "B.Cu") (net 5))
 (segment (start 102.61 35.5) (end 103.61 36.5) (width 0.2) (layer "B.Cu") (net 5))
 (segment (start 154.5 73.0808) (end 154.5 92) (width 0.2) (layer "B.Cu") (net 5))
 (segment (start 138 108.5) (end 138 133.5) (width 0.2) (layer "B.Cu") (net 5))
 (segment (start 138 133.5) (end 96.04 133.5) (width 0.2) (layer "B.Cu") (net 5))
 (segment (start 103.61 36.5) (end 103.61 41.46) (width 0.2) (layer "B.Cu") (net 5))
 (segment (start 155 69.5) (end 155.5408 70.0408) (width 0.2) (layer "F.Cu") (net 26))
 (segment (start 155.5408 70.0408) (end 162.9492 70.0408) (width 0.2) (layer "F.Cu") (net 26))
 (via (at 155 69.5) (size 0.6) (drill 0.3) (layers "F.Cu" "B.Cu") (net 26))
 (segment (start 137 65) (end 137 57) (width 0.2) (layer "B.Cu") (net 26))
 (segment (start 104.61 55) (end 103.61 56) (width 0.2) (layer "B.Cu") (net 26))
 (segment (start 154 68.5) (end 140.5 68.5) (width 0.2) (layer "B.Cu") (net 26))
 (segment (start 103.61 56) (end 103.61 60.96) (width 0.2) (layer "B.Cu") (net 26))
 (segment (start 137 57) (end 135 55) (width 0.2) (layer "B.Cu") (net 26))
 (segment (start 155 69.5) (end 154 68.5) (width 0.2) (layer "B.Cu") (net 26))
 (segment (start 140.5 68.5) (end 137 65) (width 0.2) (layer "B.Cu") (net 26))
 (segment (start 135 55) (end 104.61 55) (width 0.2) (layer "B.Cu") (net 26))
 (segment (start 154.4 68.1008) (end 155 67.5008) (width 0.2) (layer "F.Cu") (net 25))
 (segment (start 155 71) (end 154.4 70.4) (width 0.2) (layer "F.Cu") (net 25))
 (segment (start 154.4 70.4) (end 154.4 68.1008) (width 0.2) (layer "F.Cu") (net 25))
 (segment (start 155 67.5008) (end 162.9492 67.5008) (width 0.2) (layer "F.Cu") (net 25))
 (via (at 155 71) (size 0.6) (drill 0.3) (layers "F.Cu" "B.Cu") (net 25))
 (segment (start 135.25 74.5) (end 104.61 74.5) (width 0.2) (layer "B.Cu") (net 25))
 (segment (start 154 72) (end 140 72) (width 0.2) (layer "B.Cu") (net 25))
 (segment (start 155 71) (end 154 72) (width 0.2) (layer "B.Cu") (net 25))
 (segment (start 103.61 75.5) (end 103.61 80.46) (width 0.2) (layer "B.Cu") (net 25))
 (segment (start 104.61 74.5) (end 103.61 75.5) (width 0.2) (layer "B.Cu") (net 25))
 (segment (start 139.6 72.4) (end 137.35 72.4) (width 0.2) (layer "B.Cu") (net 25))
 (segment (start 140 72) (end 139.6 72.4) (width 0.2) (layer "B.Cu") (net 25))
 (segment (start 137.35 72.4) (end 135.25 74.5) (width 0.2) (layer "B.Cu") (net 25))
 (segment (start 153.692821 74.5) (end 153.692821 66.267979) (width 0.2) (layer "F.Cu") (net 24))
 (segment (start 153.692821 66.267979) (end 155 64.9608) (width 0.2) (layer "F.Cu") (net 24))
 (segment (start 155 64.9608) (end 162.9492 64.9608) (width 0.2) (layer "F.Cu") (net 24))
 (via (at 153.692821 74.5) (size 0.6) (drill 0.3) (layers "F.Cu" "B.Cu") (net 24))
 (segment (start 152.4 75.792821) (end 152.4 91.35) (width 0.2) (layer "B.Cu") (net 24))
 (segment (start 137 96) (end 135 94) (width 0.2) (layer "B.Cu") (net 24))
 (segment (start 109.57 94) (end 103.61 99.96) (width 0.2) (layer "B.Cu") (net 24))
 (segment (start 135 94) (end 109.57 94) (width 0.2) (layer "B.Cu") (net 24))
 (segment (start 152.4 91.35) (end 137 106.75) (width 0.2) (layer "B.Cu") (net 24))
 (segment (start 153.692821 74.5) (end 152.4 75.792821) (width 0.2) (layer "B.Cu") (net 24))
 (segment (start 137 106.75) (end 137 96) (width 0.2) (layer "B.Cu") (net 24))
 (segment (start 153 64.5) (end 155.0792 62.4208) (width 0.2) (layer "F.Cu") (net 6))
 (segment (start 153 77) (end 153 64.5) (width 0.2) (layer "F.Cu") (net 6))
 (segment (start 155.0792 62.4208) (end 162.9492 62.4208) (width 0.2) (layer "F.Cu") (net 6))
 (via (at 153 77) (size 0.6) (drill 0.3) (layers "F.Cu" "B.Cu") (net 6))
 (segment (start 103.61 114.39) (end 103.61 119.46) (width 0.2) (layer "B.Cu") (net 6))
 (segment (start 153 92) (end 137 108) (width 0.2) (layer "B.Cu") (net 6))
 (segment (start 153 77) (end 153 92) (width 0.2) (layer "B.Cu") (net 6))
 (segment (start 135 113.5) (end 104.5 113.5) (width 0.2) (layer "B.Cu") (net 6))
 (segment (start 104.5 113.5) (end 103.61 114.39) (width 0.2) (layer "B.Cu") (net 6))
 (segment (start 137 111.5) (end 135 113.5) (width 0.2) (layer "B.Cu") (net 6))
 (segment (start 137 108) (end 137 111.5) (width 0.2) (layer "B.Cu") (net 6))
 (segment (start 162.9492 59.8808) (end 155 59.8808) (width 0.2) (layer "F.Cu") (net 23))
 (via (at 155 59.8808) (size 0.6) (drill 0.3) (layers "F.Cu" "B.Cu") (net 23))
 (segment (start 136.5 16) (end 125 16) (width 0.2) (layer "B.Cu") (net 23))
 (segment (start 153.8808 59.8808) (end 139 45) (width 0.2) (layer "B.Cu") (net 23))
 (segment (start 139 18.5) (end 136.5 16) (width 0.2) (layer "B.Cu") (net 23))
 (segment (start 125 16) (end 123.11 17.89) (width 0.2) (layer "B.Cu") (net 23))
 (segment (start 139 45) (end 139 18.5) (width 0.2) (layer "B.Cu") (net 23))
 (segment (start 155 59.8808) (end 153.8808 59.8808) (width 0.2) (layer "B.Cu") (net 23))
 (segment (start 123.11 17.89) (end 123.11 21.96) (width 0.2) (layer "B.Cu") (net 23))
 (segment (start 138.5 38) (end 138.5 45) (width 0.2) (layer "F.Cu") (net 22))
 (segment (start 138.5 45) (end 150.8408 57.3408) (width 0.2) (layer "F.Cu") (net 22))
 (segment (start 150.8408 57.3408) (end 162.9492 57.3408) (width 0.2) (layer "F.Cu") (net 22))
 (segment (start 137.25 36.75) (end 138.5 38) (width 0.2) (layer "F.Cu") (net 22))
 (via (at 137.25 36.75) (size 0.6) (drill 0.3) (layers "F.Cu" "B.Cu") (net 22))
 (segment (start 125 35.5) (end 123.11 37.39) (width 0.2) (layer "B.Cu") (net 22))
 (segment (start 137.25 36.75) (end 136 35.5) (width 0.2) (layer "B.Cu") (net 22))
 (segment (start 136 35.5) (end 125 35.5) (width 0.2) (layer "B.Cu") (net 22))
 (segment (start 123.11 37.39) (end 123.11 41.46) (width 0.2) (layer "B.Cu") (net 22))
 (segment (start 139.434314 72) (end 139.834314 71.6) (width 0.2) (layer "B.Cu") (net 4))
 (segment (start 155.248529 70.4) (end 158.848529 74) (width 0.2) (layer "B.Cu") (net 4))
 (segment (start 153.551471 71.6) (end 154.751471 70.4) (width 0.2) (layer "B.Cu") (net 4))
 (segment (start 158.848529 74) (end 177.0684 74) (width 0.2) (layer "B.Cu") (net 4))
 (segment (start 123.11 60.96) (end 123.11 71.11) (width 0.2) (layer "B.Cu") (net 4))
 (segment (start 177.0684 74) (end 178.1892 75.1208) (width 0.2) (layer "B.Cu") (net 4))
 (segment (start 123.11 71.11) (end 124 72) (width 0.2) (layer "B.Cu") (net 4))
 (segment (start 139.834314 71.6) (end 153.551471 71.6) (width 0.2) (layer "B.Cu") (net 4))
 (segment (start 124 72) (end 139.434314 72) (width 0.2) (layer "B.Cu") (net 4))
 (segment (start 154.751471 70.4) (end 155.248529 70.4) (width 0.2) (layer "B.Cu") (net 4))
 (segment (start 180.5 77) (end 180.5 74.8916) (width 0.2) (layer "B.Cu") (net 3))
 (segment (start 180.5 74.8916) (end 178.1892 72.5808) (width 0.2) (layer "B.Cu") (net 3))
 (segment (start 124.5 92) (end 135 92) (width 0.2) (layer "B.Cu") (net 3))
 (segment (start 123.11 90.61) (end 124.5 92) (width 0.2) (layer "B.Cu") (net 3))
 (segment (start 123.11 80.46) (end 123.11 90.61) (width 0.2) (layer "B.Cu") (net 3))
 (segment (start 137 73.5) (end 137.7 72.8) (width 0.2) (layer "B.Cu") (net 3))
 (segment (start 135 92) (end 137 90) (width 0.2) (layer "B.Cu") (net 3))
 (segment (start 161 77) (end 180.5 77) (width 0.2) (layer "B.Cu") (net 3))
 (segment (start 153.765685 72.8) (end 154.584885 71.9808) (width 0.2) (layer "B.Cu") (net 3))
 (segment (start 137 90) (end 137 73.5) (width 0.2) (layer "B.Cu") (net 3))
 (segment (start 155.9808 71.9808) (end 161 77) (width 0.2) (layer "B.Cu") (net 3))
 (segment (start 137.7 72.8) (end 153.765685 72.8) (width 0.2) (layer "B.Cu") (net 3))
 (segment (start 154.584885 71.9808) (end 155.9808 71.9808) (width 0.2) (layer "B.Cu") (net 3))
 (segment (start 176.5 77.6) (end 176.5 71.73) (width 0.2) (layer "F.Cu") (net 28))
 (segment (start 137.5 105) (end 153.5 89) (width 0.2) (layer "F.Cu") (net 28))
 (segment (start 176.5 71.73) (end 178.1892 70.0408) (width 0.2) (layer "F.Cu") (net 28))
 (segment (start 153.5 89) (end 155.4 89) (width 0.2) (layer "F.Cu") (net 28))
 (segment (start 137.5 108.9) (end 137.5 105) (width 0.2) (layer "F.Cu") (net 28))
 (segment (start 136.4 110) (end 137.5 108.9) (width 0.2) (layer "F.Cu") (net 28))
 (via (at 155.4 89) (size 0.6) (drill 0.3) (layers "F.Cu" "B.Cu") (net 28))
 (via (at 136.4 110) (size 0.6) (drill 0.3) (layers "F.Cu" "B.Cu") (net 28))
 (via (at 176.5 77.6) (size 0.6) (drill 0.3) (layers "F.Cu" "B.Cu") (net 28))
 (segment (start 161 77.5) (end 176.4 77.5) (width 0.2) (layer "B.Cu") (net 28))
 (segment (start 135 111.5) (end 136.4 110.1) (width 0.2) (layer "B.Cu") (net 28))
 (segment (start 123.11 99.96) (end 123.11 110.11) (width 0.2) (layer "B.Cu") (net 28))
 (segment (start 124.5 111.5) (end 135 111.5) (width 0.2) (layer "B.Cu") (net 28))
 (segment (start 156.5 89) (end 157 88.5) (width 0.2) (layer "B.Cu") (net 28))
 (segment (start 136.4 110.1) (end 136.4 110) (width 0.2) (layer "B.Cu") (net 28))
 (segment (start 155.4 89) (end 156.5 89) (width 0.2) (layer "B.Cu") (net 28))
 (segment (start 176.4 77.5) (end 176.5 77.6) (width 0.2) (layer "B.Cu") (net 28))
 (segment (start 157 81.5) (end 161 77.5) (width 0.2) (layer "B.Cu") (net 28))
 (segment (start 157 88.5) (end 157 81.5) (width 0.2) (layer "B.Cu") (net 28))
 (segment (start 123.11 110.11) (end 124.5 111.5) (width 0.2) (layer "B.Cu") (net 28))
 (segment (start 118.5 38) (end 123 33.5) (width 0.2) (layer "F.Cu") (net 2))
 (segment (start 118.5 116.5) (end 118.5 38) (width 0.2) (layer "F.Cu") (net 2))
 (segment (start 137.5 33.5) (end 160 56) (width 0.2) (layer "F.Cu") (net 2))
 (segment (start 123 33.5) (end 128.5 33.5) (width 0.2) (layer "F.Cu") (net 2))
 (segment (start 160 56) (end 160.5 56) (width 0.2) (layer "F.Cu") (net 2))
 (via (at 128.5 33.5) (size 0.6) (drill 0.3) (layers "F.Cu" "B.Cu") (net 2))
 (via (at 160.5 56) (size 0.6) (drill 0.3) (layers "F.Cu" "B.Cu") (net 2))
 (via (at 137.5 33.5) (size 0.6) (drill 0.3) (layers "F.Cu" "B.Cu") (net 2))
 (via (at 118.5 116.5) (size 0.6) (drill 0.3) (layers "F.Cu" "B.Cu") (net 2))
 (segment (start 128.5 33.5) (end 137.5 33.5) (width 0.2) (layer "B.Cu") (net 2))
 (segment (start 160.5 56) (end 170.784035 56) (width 0.2) (layer "B.Cu") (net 2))
 (segment (start 177.0892 66.4008) (end 178.1892 67.5008) (width 0.2) (layer "B.Cu") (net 2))
 (segment (start 170.784035 56) (end 177.0892 62.305165) (width 0.2) (layer "B.Cu") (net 2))
 (segment (start 177.0892 62.305165) (end 177.0892 66.4008) (width 0.2) (layer "B.Cu") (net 2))
 (segment (start 121.46 119.46) (end 118.5 116.5) (width 0.2) (layer "B.Cu") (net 2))
 (segment (start 123.11 119.46) (end 121.46 119.46) (width 0.2) (layer "B.Cu") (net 2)))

